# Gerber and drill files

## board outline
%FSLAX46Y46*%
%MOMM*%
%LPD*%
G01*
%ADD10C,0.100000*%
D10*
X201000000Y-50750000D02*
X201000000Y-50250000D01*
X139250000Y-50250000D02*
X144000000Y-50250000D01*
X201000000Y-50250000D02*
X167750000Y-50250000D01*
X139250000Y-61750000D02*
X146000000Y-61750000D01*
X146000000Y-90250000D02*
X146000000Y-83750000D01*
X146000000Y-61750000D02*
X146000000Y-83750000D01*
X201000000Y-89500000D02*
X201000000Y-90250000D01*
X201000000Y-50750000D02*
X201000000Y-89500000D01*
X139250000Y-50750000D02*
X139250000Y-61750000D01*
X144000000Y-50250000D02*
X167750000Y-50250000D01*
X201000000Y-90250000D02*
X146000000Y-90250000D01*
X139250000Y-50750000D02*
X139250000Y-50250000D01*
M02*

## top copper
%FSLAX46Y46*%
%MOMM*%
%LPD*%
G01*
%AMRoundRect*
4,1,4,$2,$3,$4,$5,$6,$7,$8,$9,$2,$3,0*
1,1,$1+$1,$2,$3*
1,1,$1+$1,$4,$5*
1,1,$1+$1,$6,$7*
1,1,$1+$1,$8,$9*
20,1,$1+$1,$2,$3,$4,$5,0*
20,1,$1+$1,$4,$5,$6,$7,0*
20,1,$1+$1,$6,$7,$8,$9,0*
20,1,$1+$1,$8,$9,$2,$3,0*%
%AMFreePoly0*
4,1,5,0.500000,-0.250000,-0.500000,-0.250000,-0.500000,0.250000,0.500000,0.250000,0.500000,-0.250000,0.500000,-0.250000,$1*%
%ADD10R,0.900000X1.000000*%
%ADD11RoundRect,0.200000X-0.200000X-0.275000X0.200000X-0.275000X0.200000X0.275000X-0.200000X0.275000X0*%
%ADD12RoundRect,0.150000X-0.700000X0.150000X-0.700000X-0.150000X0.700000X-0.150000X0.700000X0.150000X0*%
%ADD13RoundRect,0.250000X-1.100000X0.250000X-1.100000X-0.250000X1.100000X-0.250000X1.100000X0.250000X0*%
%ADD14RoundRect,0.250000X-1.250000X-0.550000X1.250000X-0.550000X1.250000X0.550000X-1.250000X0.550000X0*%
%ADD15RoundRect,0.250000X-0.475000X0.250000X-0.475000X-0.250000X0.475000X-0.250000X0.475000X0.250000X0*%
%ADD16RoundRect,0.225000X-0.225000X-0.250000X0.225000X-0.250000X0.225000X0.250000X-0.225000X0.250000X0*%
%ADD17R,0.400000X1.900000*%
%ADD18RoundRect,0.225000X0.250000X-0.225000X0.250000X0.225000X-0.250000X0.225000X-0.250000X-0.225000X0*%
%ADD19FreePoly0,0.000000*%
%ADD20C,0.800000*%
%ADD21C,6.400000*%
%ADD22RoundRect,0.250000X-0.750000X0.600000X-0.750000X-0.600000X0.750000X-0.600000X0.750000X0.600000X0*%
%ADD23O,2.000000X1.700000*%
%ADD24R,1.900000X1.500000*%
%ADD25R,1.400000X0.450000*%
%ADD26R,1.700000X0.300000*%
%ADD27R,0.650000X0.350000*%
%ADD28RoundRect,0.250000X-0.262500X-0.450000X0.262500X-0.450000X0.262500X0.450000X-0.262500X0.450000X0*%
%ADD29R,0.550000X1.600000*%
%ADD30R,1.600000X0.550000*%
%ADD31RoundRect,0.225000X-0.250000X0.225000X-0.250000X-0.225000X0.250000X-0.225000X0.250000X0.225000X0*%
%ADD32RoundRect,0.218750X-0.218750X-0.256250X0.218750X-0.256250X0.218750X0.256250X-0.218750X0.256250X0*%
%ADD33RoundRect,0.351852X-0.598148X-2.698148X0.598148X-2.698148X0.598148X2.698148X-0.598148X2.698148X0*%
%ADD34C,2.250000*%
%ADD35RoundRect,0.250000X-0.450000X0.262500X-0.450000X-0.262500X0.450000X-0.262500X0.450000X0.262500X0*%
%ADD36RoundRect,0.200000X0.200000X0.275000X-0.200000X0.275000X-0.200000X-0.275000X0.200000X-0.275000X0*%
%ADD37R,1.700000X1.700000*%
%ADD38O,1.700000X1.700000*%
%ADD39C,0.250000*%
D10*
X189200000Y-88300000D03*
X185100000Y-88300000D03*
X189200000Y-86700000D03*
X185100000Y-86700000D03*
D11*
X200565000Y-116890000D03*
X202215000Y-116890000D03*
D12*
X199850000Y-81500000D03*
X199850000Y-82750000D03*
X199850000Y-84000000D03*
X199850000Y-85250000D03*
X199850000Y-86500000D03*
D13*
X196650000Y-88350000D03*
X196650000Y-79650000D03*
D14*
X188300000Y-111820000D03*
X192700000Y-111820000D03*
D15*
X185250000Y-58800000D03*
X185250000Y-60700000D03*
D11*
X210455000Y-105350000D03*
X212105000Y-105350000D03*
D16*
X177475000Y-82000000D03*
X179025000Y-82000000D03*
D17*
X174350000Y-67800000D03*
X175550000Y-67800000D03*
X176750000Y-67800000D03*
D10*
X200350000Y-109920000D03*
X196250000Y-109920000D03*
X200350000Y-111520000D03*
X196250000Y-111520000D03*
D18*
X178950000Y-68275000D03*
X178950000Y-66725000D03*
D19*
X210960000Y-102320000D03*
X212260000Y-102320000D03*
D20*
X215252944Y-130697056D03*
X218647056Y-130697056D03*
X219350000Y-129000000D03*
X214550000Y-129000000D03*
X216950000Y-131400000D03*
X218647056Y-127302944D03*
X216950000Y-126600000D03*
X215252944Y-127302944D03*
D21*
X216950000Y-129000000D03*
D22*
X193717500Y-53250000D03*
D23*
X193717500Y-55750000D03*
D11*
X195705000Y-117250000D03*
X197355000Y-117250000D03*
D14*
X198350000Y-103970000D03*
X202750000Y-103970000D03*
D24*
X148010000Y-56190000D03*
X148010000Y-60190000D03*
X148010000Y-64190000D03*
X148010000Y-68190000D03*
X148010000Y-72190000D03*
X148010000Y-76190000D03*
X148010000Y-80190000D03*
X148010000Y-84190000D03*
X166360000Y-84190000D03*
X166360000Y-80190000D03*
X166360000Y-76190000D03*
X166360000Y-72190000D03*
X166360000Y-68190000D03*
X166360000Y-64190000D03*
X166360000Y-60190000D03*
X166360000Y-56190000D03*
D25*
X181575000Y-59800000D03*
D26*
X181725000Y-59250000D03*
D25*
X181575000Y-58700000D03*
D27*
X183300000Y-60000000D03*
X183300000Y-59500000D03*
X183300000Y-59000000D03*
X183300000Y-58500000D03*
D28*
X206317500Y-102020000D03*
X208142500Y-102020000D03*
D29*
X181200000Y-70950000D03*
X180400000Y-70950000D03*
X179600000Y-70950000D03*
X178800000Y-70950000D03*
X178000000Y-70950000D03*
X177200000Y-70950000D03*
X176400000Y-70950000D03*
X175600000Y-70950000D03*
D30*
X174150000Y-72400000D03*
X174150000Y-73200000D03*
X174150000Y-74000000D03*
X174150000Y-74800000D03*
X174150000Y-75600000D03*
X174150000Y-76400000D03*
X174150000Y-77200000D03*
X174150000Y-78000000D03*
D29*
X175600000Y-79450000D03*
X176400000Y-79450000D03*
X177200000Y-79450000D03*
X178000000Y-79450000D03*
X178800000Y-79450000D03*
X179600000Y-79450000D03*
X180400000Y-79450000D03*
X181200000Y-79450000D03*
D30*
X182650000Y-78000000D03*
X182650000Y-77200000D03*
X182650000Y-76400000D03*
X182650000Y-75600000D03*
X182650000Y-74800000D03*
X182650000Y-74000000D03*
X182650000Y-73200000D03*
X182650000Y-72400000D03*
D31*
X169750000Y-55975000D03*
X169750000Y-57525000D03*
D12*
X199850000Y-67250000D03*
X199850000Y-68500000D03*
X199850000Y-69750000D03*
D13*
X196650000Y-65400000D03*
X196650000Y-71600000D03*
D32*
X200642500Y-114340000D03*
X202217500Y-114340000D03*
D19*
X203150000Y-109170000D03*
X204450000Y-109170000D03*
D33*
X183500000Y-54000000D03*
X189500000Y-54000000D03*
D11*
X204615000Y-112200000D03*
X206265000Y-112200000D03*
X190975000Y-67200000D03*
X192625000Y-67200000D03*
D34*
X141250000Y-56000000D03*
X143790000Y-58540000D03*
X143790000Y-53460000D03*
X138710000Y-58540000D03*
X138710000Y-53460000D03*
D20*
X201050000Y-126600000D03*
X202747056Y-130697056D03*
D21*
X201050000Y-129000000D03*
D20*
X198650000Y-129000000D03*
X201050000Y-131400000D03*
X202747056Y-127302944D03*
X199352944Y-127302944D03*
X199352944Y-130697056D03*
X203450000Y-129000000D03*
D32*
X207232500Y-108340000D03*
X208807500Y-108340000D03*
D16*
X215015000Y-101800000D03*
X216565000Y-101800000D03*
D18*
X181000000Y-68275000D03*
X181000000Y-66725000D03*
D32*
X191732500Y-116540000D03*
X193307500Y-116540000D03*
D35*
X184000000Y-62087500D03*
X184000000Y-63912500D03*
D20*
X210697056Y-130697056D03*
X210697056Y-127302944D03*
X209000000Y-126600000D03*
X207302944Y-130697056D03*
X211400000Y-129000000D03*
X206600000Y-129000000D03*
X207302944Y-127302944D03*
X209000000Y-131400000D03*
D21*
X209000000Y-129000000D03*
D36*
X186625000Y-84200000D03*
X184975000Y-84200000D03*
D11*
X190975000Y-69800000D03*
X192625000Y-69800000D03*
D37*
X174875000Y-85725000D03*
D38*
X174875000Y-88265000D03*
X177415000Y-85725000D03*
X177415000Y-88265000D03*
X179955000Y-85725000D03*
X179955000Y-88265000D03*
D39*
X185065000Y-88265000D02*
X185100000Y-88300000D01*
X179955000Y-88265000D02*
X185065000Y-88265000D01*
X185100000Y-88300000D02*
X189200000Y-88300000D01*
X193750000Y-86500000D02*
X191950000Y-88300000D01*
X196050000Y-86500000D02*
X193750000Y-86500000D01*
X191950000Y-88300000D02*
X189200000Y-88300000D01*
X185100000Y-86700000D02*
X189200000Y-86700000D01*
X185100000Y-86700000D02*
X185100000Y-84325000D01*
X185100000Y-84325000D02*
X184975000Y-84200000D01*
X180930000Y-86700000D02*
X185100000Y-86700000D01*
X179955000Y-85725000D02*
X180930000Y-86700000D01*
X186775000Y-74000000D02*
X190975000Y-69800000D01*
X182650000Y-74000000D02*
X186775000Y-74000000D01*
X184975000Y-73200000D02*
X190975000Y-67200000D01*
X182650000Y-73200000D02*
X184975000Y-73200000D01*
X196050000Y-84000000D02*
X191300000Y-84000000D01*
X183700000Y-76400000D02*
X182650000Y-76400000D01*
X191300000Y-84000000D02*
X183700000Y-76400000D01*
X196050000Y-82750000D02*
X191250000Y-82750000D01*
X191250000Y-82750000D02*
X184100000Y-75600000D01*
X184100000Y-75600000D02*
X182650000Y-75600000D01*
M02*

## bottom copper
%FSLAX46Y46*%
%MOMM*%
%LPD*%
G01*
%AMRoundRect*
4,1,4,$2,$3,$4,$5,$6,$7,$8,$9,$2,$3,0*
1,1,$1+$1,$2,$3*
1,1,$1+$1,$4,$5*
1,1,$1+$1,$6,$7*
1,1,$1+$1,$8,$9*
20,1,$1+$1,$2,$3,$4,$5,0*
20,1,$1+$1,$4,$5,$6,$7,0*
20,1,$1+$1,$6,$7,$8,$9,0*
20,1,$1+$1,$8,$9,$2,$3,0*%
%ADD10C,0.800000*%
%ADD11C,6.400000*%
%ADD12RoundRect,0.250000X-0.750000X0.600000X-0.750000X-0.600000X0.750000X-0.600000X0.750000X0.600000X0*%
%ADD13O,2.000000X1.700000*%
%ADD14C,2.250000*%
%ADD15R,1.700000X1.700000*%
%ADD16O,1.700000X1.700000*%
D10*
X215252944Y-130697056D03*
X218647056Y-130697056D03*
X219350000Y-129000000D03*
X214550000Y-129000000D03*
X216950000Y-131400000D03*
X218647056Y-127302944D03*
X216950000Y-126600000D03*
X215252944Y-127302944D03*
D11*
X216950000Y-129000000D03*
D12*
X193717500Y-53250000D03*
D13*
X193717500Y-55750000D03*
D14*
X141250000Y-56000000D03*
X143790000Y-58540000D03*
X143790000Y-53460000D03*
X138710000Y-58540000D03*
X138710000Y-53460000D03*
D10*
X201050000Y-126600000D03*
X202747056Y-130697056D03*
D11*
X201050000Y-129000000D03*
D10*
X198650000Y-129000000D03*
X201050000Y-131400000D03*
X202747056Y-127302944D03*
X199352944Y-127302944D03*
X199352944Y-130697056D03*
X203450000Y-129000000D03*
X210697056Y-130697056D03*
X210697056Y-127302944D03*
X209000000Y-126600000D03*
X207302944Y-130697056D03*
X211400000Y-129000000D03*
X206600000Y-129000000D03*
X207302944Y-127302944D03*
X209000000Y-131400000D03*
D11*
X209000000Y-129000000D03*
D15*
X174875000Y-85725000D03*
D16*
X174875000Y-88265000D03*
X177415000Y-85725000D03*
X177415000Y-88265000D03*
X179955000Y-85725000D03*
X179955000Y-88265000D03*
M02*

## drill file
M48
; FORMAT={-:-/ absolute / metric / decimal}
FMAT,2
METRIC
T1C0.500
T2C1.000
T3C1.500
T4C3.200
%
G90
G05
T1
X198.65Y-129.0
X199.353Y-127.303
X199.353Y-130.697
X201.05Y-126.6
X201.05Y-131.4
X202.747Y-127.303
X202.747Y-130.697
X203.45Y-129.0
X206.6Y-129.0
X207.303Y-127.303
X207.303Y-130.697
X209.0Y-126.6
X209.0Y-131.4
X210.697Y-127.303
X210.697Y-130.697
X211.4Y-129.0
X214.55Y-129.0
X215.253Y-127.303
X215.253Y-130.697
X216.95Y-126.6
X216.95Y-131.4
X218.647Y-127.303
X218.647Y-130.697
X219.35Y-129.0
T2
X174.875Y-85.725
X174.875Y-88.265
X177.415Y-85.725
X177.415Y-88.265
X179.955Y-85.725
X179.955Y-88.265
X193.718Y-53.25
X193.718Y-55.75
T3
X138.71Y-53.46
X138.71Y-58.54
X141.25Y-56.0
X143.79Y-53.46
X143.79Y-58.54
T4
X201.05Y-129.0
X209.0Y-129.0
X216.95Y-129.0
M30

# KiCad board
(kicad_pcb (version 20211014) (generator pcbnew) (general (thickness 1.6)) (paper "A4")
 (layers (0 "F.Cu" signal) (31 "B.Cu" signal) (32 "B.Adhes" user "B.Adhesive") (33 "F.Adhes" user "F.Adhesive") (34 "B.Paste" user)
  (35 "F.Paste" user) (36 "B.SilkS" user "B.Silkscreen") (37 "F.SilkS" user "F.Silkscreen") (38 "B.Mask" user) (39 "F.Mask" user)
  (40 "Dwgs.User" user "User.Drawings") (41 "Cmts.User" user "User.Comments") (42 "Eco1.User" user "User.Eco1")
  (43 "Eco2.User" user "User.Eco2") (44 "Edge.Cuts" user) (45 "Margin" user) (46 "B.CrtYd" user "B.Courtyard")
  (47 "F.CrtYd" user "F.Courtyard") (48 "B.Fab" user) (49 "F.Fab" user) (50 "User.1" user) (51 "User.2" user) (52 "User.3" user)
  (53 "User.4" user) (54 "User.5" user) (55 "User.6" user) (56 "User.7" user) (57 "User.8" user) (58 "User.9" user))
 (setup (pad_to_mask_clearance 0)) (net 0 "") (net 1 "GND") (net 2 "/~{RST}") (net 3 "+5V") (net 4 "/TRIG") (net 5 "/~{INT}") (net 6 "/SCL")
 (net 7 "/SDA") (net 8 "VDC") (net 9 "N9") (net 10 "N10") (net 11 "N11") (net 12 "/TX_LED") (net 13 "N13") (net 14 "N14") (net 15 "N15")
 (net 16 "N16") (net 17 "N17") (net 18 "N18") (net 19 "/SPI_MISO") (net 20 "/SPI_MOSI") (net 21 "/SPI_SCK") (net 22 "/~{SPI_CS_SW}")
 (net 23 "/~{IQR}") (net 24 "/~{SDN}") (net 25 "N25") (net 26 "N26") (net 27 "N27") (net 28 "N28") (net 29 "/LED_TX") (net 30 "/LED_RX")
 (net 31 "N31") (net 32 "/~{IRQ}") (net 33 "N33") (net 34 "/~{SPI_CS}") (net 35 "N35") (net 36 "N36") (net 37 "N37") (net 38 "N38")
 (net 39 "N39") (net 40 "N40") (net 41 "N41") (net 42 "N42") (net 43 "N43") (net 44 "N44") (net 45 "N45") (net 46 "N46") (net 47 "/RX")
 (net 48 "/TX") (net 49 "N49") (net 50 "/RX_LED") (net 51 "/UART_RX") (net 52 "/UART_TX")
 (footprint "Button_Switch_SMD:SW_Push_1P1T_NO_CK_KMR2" (layer "F.Cu") (at 187.15 87.5 180)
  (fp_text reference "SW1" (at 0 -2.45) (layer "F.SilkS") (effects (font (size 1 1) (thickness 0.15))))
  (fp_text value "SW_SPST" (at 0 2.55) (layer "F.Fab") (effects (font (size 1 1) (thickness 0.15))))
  (pad "1" smd rect (at -2.05 -0.8 180) (size 0.9 1) (layers "F.Cu" "F.Paste" "F.Mask") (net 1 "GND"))
  (pad "1" smd rect (at 2.05 -0.8 180) (size 0.9 1) (layers "F.Cu" "F.Paste" "F.Mask") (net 1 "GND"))
  (pad "2" smd rect (at -2.05 0.8 180) (size 0.9 1) (layers "F.Cu" "F.Paste" "F.Mask") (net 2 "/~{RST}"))
  (pad "2" smd rect (at 2.05 0.8 180) (size 0.9 1) (layers "F.Cu" "F.Paste" "F.Mask") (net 2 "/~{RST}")))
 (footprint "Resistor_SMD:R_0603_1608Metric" (layer "F.Cu") (at 201.39 116.89)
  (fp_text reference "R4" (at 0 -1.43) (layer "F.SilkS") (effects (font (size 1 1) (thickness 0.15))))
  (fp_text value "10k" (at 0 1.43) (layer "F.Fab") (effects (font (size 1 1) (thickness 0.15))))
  (pad "1" smd roundrect (at -0.825 0) (size 0.8 0.95) (layers "F.Cu" "F.Paste" "F.Mask") (roundrect_rratio 0.25) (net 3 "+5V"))
  (pad "2" smd roundrect (at 0.825 0) (size 0.8 0.95) (layers "F.Cu" "F.Paste" "F.Mask") (roundrect_rratio 0.25) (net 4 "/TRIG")))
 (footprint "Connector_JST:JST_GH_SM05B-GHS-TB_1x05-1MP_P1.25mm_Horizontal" (layer "F.Cu") (at 198 84 -90)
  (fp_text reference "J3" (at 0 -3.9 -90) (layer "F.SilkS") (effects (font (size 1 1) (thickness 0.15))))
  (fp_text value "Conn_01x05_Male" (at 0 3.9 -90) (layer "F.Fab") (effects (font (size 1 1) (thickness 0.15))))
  (pad "1" smd roundrect (at -2.5 -1.85 270) (size 0.6 1.7) (layers "F.Cu" "F.Paste" "F.Mask") (roundrect_rratio 0.25) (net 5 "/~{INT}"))
  (pad "2" smd roundrect (at -1.25 -1.85 270) (size 0.6 1.7) (layers "F.Cu" "F.Paste" "F.Mask") (roundrect_rratio 0.25) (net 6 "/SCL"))
  (pad "3" smd roundrect (at 0 -1.85 270) (size 0.6 1.7) (layers "F.Cu" "F.Paste" "F.Mask") (roundrect_rratio 0.25) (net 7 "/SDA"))
  (pad "4" smd roundrect (at 1.25 -1.85 270) (size 0.6 1.7) (layers "F.Cu" "F.Paste" "F.Mask") (roundrect_rratio 0.25) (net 3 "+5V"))
  (pad "5" smd roundrect (at 2.5 -1.85 270) (size 0.6 1.7) (layers "F.Cu" "F.Paste" "F.Mask") (roundrect_rratio 0.25) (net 1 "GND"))
  (pad "MP" smd roundrect (at 4.35 1.35 270) (size 1 2.7) (layers "F.Cu" "F.Paste" "F.Mask") (roundrect_rratio 0.25))
  (pad "MP" smd roundrect (at -4.35 1.35 270) (size 1 2.7) (layers "F.Cu" "F.Paste" "F.Mask") (roundrect_rratio 0.25)))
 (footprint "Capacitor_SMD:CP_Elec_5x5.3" (layer "F.Cu") (at 190.5 111.82)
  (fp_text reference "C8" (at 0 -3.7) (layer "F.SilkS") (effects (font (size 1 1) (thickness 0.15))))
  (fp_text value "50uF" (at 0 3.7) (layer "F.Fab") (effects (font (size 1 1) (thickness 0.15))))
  (pad "1" smd roundrect (at -2.2 0) (size 3 1.6) (layers "F.Cu" "F.Paste" "F.Mask") (roundrect_rratio 0.15625) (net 3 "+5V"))
  (pad "2" smd roundrect (at 2.2 0) (size 3 1.6) (layers "F.Cu" "F.Paste" "F.Mask") (roundrect_rratio 0.15625) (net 1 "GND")))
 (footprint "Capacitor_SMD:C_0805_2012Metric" (layer "F.Cu") (at 185.25 59.75 -90)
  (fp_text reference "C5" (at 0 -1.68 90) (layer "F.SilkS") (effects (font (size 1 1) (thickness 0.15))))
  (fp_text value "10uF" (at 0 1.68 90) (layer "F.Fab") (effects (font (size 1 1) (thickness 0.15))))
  (pad "1" smd roundrect (at -0.95 0 270) (size 1 1.45) (layers "F.Cu" "F.Paste" "F.Mask") (roundrect_rratio 0.25) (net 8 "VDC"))
  (pad "2" smd roundrect (at 0.95 0 270) (size 1 1.45) (layers "F.Cu" "F.Paste" "F.Mask") (roundrect_rratio 0.25) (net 1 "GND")))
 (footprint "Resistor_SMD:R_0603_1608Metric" (layer "F.Cu") (at 211.28 105.35)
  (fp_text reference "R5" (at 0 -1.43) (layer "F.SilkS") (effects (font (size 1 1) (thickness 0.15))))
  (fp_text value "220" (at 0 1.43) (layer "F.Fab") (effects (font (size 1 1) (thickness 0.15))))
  (pad "1" smd roundrect (at -0.825 0) (size 0.8 0.95) (layers "F.Cu" "F.Paste" "F.Mask") (roundrect_rratio 0.25) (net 3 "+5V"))
  (pad "2" smd roundrect (at 0.825 0) (size 0.8 0.95) (layers "F.Cu" "F.Paste" "F.Mask") (roundrect_rratio 0.25) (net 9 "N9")))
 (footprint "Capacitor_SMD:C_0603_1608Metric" (layer "F.Cu") (at 178.25 82)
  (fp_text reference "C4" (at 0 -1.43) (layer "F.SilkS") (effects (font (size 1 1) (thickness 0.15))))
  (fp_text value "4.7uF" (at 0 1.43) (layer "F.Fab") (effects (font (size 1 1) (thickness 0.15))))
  (pad "1" smd roundrect (at -0.775 0) (size 0.9 0.95) (layers "F.Cu" "F.Paste" "F.Mask") (roundrect_rratio 0.25) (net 3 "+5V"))
  (pad "2" smd roundrect (at 0.775 0) (size 0.9 0.95) (layers "F.Cu" "F.Paste" "F.Mask") (roundrect_rratio 0.25) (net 1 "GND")))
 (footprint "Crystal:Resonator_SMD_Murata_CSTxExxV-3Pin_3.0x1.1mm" (layer "F.Cu") (at 175.55 67.8)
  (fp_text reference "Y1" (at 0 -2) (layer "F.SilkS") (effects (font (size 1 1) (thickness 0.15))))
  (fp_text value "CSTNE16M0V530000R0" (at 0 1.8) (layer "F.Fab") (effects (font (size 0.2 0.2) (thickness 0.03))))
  (pad "1" smd rect (at -1.2 0) (size 0.4 1.9) (layers "F.Cu" "F.Paste" "F.Mask") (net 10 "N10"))
  (pad "2" smd rect (at 0 0) (size 0.4 1.9) (layers "F.Cu" "F.Paste" "F.Mask") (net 1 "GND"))
  (pad "3" smd rect (at 1.2 0) (size 0.4 1.9) (layers "F.Cu" "F.Paste" "F.Mask") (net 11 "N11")))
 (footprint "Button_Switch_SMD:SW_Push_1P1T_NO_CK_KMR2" (layer "F.Cu") (at 198.3 110.72)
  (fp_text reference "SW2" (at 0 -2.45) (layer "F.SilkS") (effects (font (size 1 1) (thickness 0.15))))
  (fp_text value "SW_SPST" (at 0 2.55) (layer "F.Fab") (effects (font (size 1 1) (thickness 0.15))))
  (pad "1" smd rect (at 2.05 -0.8) (size 0.9 1) (layers "F.Cu" "F.Paste" "F.Mask") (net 1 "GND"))
  (pad "1" smd rect (at -2.05 -0.8) (size 0.9 1) (layers "F.Cu" "F.Paste" "F.Mask") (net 1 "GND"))
  (pad "2" smd rect (at 2.05 0.8) (size 0.9 1) (layers "F.Cu" "F.Paste" "F.Mask") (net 4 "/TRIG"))
  (pad "2" smd rect (at -2.05 0.8) (size 0.9 1) (layers "F.Cu" "F.Paste" "F.Mask") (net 4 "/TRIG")))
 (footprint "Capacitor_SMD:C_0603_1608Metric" (layer "F.Cu") (at 178.95 67.5 90)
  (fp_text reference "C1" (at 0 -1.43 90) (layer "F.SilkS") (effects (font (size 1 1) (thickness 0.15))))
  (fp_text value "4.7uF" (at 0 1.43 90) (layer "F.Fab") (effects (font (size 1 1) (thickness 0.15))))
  (pad "1" smd roundrect (at -0.775 0 90) (size 0.9 0.95) (layers "F.Cu" "F.Paste" "F.Mask") (roundrect_rratio 0.25) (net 3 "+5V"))
  (pad "2" smd roundrect (at 0.775 0 90) (size 0.9 0.95) (layers "F.Cu" "F.Paste" "F.Mask") (roundrect_rratio 0.25) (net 1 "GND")))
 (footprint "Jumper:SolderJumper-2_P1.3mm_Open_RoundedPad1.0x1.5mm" (layer "F.Cu") (at 211.61 102.32)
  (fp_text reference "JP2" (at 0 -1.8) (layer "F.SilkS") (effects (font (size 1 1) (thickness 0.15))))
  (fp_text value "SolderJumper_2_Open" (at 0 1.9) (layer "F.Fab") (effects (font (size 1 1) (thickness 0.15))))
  (pad "1" smd custom (at -0.65 0) (size 1 0.5) (layers "F.Cu" "F.Mask") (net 3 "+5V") (zone_connect 2)
   (options (clearance outline) (anchor rect)) (primitives))
  (pad "2" smd custom (at 0.65 0) (size 1 0.5) (layers "F.Cu" "F.Mask") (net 8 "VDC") (zone_connect 2)
   (options (clearance outline) (anchor rect)) (primitives)))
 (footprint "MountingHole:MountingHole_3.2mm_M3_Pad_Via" (layer "F.Cu") (at 216.95 129)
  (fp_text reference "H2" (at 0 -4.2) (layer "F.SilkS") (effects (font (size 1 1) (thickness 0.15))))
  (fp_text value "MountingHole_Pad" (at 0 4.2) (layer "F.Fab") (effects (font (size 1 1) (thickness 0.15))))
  (pad "1" thru_hole circle (at -1.697056 1.697056) (size 0.8 0.8) (drill 0.5) (layers *.Cu *.Mask) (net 1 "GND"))
  (pad "1" thru_hole circle (at 1.697056 1.697056) (size 0.8 0.8) (drill 0.5) (layers *.Cu *.Mask) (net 1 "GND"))
  (pad "1" thru_hole circle (at 2.4 0) (size 0.8 0.8) (drill 0.5) (layers *.Cu *.Mask) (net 1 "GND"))
  (pad "1" thru_hole circle (at -2.4 0) (size 0.8 0.8) (drill 0.5) (layers *.Cu *.Mask) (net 1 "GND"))
  (pad "1" thru_hole circle (at 0 2.4) (size 0.8 0.8) (drill 0.5) (layers *.Cu *.Mask) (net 1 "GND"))
  (pad "1" thru_hole circle (at 1.697056 -1.697056) (size 0.8 0.8) (drill 0.5) (layers *.Cu *.Mask) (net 1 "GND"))
  (pad "1" thru_hole circle (at 0 -2.4) (size 0.8 0.8) (drill 0.5) (layers *.Cu *.Mask) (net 1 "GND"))
  (pad "1" thru_hole circle (at -1.697056 -1.697056) (size 0.8 0.8) (drill 0.5) (layers *.Cu *.Mask) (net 1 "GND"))
  (pad "1" thru_hole circle (at 0 0) (size 6.4 6.4) (drill 3.2) (layers *.Cu *.Mask) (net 1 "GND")))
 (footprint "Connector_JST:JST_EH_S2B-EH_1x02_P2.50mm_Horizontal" (layer "F.Cu") (at 193.7175 53.25 -90)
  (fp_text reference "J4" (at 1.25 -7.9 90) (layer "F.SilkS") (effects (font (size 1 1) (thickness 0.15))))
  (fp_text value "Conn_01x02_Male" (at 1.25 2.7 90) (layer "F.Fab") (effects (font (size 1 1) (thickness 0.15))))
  (pad "1" thru_hole roundrect (at 0 0 270) (size 1.7 2) (drill 1) (layers *.Cu *.Mask) (roundrect_rratio 0.147059) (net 3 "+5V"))
  (pad "2" thru_hole oval (at 2.5 0 270) (size 1.7 2) (drill 1) (layers *.Cu *.Mask) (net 1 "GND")))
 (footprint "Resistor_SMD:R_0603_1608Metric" (layer "F.Cu") (at 196.53 117.25)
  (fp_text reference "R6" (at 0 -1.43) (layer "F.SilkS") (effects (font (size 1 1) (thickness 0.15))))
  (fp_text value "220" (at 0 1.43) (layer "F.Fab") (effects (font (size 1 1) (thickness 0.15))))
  (pad "1" smd roundrect (at -0.825 0) (size 0.8 0.95) (layers "F.Cu" "F.Paste" "F.Mask") (roundrect_rratio 0.25) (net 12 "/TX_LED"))
  (pad "2" smd roundrect (at 0.825 0) (size 0.8 0.95) (layers "F.Cu" "F.Paste" "F.Mask") (roundrect_rratio 0.25) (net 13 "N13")))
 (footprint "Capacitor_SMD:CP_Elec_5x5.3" (layer "F.Cu") (at 200.55 103.97)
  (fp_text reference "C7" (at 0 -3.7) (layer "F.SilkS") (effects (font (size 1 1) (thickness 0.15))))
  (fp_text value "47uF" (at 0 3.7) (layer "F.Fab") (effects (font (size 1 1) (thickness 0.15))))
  (pad "1" smd roundrect (at -2.2 0) (size 3 1.6) (layers "F.Cu" "F.Paste" "F.Mask") (roundrect_rratio 0.15625) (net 3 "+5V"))
  (pad "2" smd roundrect (at 2.2 0) (size 3 1.6) (layers "F.Cu" "F.Paste" "F.Mask") (roundrect_rratio 0.15625) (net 1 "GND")))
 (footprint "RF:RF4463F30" (layer "F.Cu") (at 157.21 70.19)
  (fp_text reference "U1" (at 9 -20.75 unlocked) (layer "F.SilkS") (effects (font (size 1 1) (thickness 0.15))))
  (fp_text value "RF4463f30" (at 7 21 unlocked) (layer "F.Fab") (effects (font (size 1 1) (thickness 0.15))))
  (pad "1" smd rect (at -9.2 -14 270) (size 1.5 1.9) (layers "F.Cu" "F.Paste" "F.Mask") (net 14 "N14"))
  (pad "2" smd rect (at -9.2 -10 270) (size 1.5 1.9) (layers "F.Cu" "F.Paste" "F.Mask") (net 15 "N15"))
  (pad "3" smd rect (at -9.2 -6 90) (size 1.5 1.9) (layers "F.Cu" "F.Paste" "F.Mask") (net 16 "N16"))
  (pad "4" smd rect (at -9.2 -2 90) (size 1.5 1.9) (layers "F.Cu" "F.Paste" "F.Mask") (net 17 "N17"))
  (pad "5" smd rect (at -9.2 2 270) (size 1.5 1.9) (layers "F.Cu" "F.Paste" "F.Mask") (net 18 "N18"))
  (pad "6" smd rect (at -9.2 6 90) (size 1.5 1.9) (layers "F.Cu" "F.Paste" "F.Mask") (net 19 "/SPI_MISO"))
  (pad "7" smd rect (at -9.2 10 90) (size 1.5 1.9) (layers "F.Cu" "F.Paste" "F.Mask") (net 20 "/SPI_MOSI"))
  (pad "8" smd rect (at -9.2 14 90) (size 1.5 1.9) (layers "F.Cu" "F.Paste" "F.Mask") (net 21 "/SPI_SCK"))
  (pad "9" smd rect (at 9.15 14 90) (size 1.5 1.9) (layers "F.Cu" "F.Paste" "F.Mask") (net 1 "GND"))
  (pad "10" smd rect (at 9.15 10 90) (size 1.5 1.9) (layers "F.Cu" "F.Paste" "F.Mask") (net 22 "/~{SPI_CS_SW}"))
  (pad "11" smd rect (at 9.15 6 90) (size 1.5 1.9) (layers "F.Cu" "F.Paste" "F.Mask") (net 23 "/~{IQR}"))
  (pad "12" smd rect (at 9.15 2 90) (size 1.5 1.9) (layers "F.Cu" "F.Paste" "F.Mask") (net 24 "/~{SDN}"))
  (pad "13" smd rect (at 9.15 -2 90) (size 1.5 1.9) (layers "F.Cu" "F.Paste" "F.Mask") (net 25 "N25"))
  (pad "14" smd rect (at 9.15 -6 90) (size 1.5 1.9) (layers "F.Cu" "F.Paste" "F.Mask") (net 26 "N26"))
  (pad "15" smd rect (at 9.15 -10 90) (size 1.5 1.9) (layers "F.Cu" "F.Paste" "F.Mask") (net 1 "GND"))
  (pad "16" smd rect (at 9.15 -14 90) (size 1.5 1.9) (layers "F.Cu" "F.Paste" "F.Mask") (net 3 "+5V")))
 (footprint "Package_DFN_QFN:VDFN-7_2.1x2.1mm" (layer "F.Cu") (at 182.25 59.25)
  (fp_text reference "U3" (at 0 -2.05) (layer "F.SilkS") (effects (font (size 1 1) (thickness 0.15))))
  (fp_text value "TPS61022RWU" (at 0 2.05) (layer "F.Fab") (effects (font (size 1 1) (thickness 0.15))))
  (pad "1" smd rect (at -0.675 0.55) (size 1.4 0.45) (layers "F.Cu" "F.Paste" "F.Mask") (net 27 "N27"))
  (pad "2" smd rect (at -0.525 0) (size 1.7 0.3) (layers "F.Cu" "F.Paste" "F.Mask") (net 8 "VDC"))
  (pad "3" smd rect (at -0.675 -0.55) (size 1.4 0.45) (layers "F.Cu" "F.Paste" "F.Mask") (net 1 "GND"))
  (pad "5" smd rect (at 1.05 0.75) (size 0.65 0.35) (layers "F.Cu" "F.Paste" "F.Mask") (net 1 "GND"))
  (pad "6" smd rect (at 1.05 0.25) (size 0.65 0.35) (layers "F.Cu" "F.Paste" "F.Mask") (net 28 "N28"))
  (pad "7" smd rect (at 1.05 -0.25) (size 0.65 0.35) (layers "F.Cu" "F.Paste" "F.Mask") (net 3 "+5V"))
  (pad "8" smd rect (at 1.05 -0.75) (size 0.65 0.35) (layers "F.Cu" "F.Paste" "F.Mask")))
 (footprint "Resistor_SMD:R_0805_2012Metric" (layer "F.Cu") (at 207.23 102.02)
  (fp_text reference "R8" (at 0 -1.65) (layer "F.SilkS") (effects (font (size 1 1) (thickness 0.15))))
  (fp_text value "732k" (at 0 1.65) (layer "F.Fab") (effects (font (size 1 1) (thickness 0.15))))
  (pad "1" smd roundrect (at -0.9125 0) (size 1.025 1.4) (layers "F.Cu" "F.Paste" "F.Mask") (roundrect_rratio 0.243902) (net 3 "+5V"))
  (pad "2" smd roundrect (at 0.9125 0) (size 1.025 1.4) (layers "F.Cu" "F.Paste" "F.Mask") (roundrect_rratio 0.243902) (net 27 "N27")))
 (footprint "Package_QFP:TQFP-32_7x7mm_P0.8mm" (layer "F.Cu") (at 178.4 75.2 -90)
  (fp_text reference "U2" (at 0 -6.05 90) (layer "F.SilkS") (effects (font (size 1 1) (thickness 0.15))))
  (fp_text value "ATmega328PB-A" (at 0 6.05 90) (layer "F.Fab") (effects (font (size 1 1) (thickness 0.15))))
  (pad "1" smd rect (at -4.25 -2.8 270) (size 1.6 0.55) (layers "F.Cu" "F.Paste" "F.Mask") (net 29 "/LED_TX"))
  (pad "2" smd rect (at -4.25 -2 270) (size 1.6 0.55) (layers "F.Cu" "F.Paste" "F.Mask") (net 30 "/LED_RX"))
  (pad "3" smd rect (at -4.25 -1.2 270) (size 1.6 0.55) (layers "F.Cu" "F.Paste" "F.Mask") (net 20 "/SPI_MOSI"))
  (pad "4" smd rect (at -4.25 -0.4 270) (size 1.6 0.55) (layers "F.Cu" "F.Paste" "F.Mask") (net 3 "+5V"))
  (pad "5" smd rect (at -4.25 0.4 270) (size 1.6 0.55) (layers "F.Cu" "F.Paste" "F.Mask") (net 1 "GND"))
  (pad "6" smd rect (at -4.25 1.2 270) (size 1.6 0.55) (layers "F.Cu" "F.Paste" "F.Mask") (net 19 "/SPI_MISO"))
  (pad "7" smd rect (at -4.25 2 270) (size 1.6 0.55) (layers "F.Cu" "F.Paste" "F.Mask") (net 11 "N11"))
  (pad "8" smd rect (at -4.25 2.8 270) (size 1.6 0.55) (layers "F.Cu" "F.Paste" "F.Mask") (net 10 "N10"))
  (pad "9" smd rect (at -2.8 4.25) (size 1.6 0.55) (layers "F.Cu" "F.Paste" "F.Mask") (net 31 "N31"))
  (pad "10" smd rect (at -2 4.25) (size 1.6 0.55) (layers "F.Cu" "F.Paste" "F.Mask") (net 24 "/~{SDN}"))
  (pad "11" smd rect (at -1.2 4.25) (size 1.6 0.55) (layers "F.Cu" "F.Paste" "F.Mask") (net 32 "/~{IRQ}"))
  (pad "12" smd rect (at -0.4 4.25) (size 1.6 0.55) (layers "F.Cu" "F.Paste" "F.Mask") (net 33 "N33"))
  (pad "13" smd rect (at 0.4 4.25) (size 1.6 0.55) (layers "F.Cu" "F.Paste" "F.Mask") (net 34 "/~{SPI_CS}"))
  (pad "14" smd rect (at 1.2 4.25) (size 1.6 0.55) (layers "F.Cu" "F.Paste" "F.Mask") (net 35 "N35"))
  (pad "15" smd rect (at 2 4.25) (size 1.6 0.55) (layers "F.Cu" "F.Paste" "F.Mask") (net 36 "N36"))
  (pad "16" smd rect (at 2.8 4.25) (size 1.6 0.55) (layers "F.Cu" "F.Paste" "F.Mask") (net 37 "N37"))
  (pad "17" smd rect (at 4.25 2.8 270) (size 1.6 0.55) (layers "F.Cu" "F.Paste" "F.Mask") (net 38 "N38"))
  (pad "18" smd rect (at 4.25 2 270) (size 1.6 0.55) (layers "F.Cu" "F.Paste" "F.Mask") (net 3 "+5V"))
  (pad "19" smd rect (at 4.25 1.2 270) (size 1.6 0.55) (layers "F.Cu" "F.Paste" "F.Mask") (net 21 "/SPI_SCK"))
  (pad "20" smd rect (at 4.25 0.4 270) (size 1.6 0.55) (layers "F.Cu" "F.Paste" "F.Mask") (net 3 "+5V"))
  (pad "21" smd rect (at 4.25 -0.4 270) (size 1.6 0.55) (layers "F.Cu" "F.Paste" "F.Mask") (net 1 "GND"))
  (pad "22" smd rect (at 4.25 -1.2 270) (size 1.6 0.55) (layers "F.Cu" "F.Paste" "F.Mask") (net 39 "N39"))
  (pad "23" smd rect (at 4.25 -2 270) (size 1.6 0.55) (layers "F.Cu" "F.Paste" "F.Mask") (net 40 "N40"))
  (pad "24" smd rect (at 4.25 -2.8 270) (size 1.6 0.55) (layers "F.Cu" "F.Paste" "F.Mask") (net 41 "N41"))
  (pad "25" smd rect (at 2.8 -4.25) (size 1.6 0.55) (layers "F.Cu" "F.Paste" "F.Mask") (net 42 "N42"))
  (pad "26" smd rect (at 2 -4.25) (size 1.6 0.55) (layers "F.Cu" "F.Paste" "F.Mask") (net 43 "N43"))
  (pad "27" smd rect (at 1.2 -4.25) (size 1.6 0.55) (layers "F.Cu" "F.Paste" "F.Mask") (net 7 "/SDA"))
  (pad "28" smd rect (at 0.4 -4.25) (size 1.6 0.55) (layers "F.Cu" "F.Paste" "F.Mask") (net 6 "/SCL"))
  (pad "29" smd rect (at -0.4 -4.25) (size 1.6 0.55) (layers "F.Cu" "F.Paste" "F.Mask") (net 2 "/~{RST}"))
  (pad "30" smd rect (at -1.2 -4.25) (size 1.6 0.55) (layers "F.Cu" "F.Paste" "F.Mask") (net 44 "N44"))
  (pad "31" smd rect (at -2 -4.25) (size 1.6 0.55) (layers "F.Cu" "F.Paste" "F.Mask") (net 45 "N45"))
  (pad "32" smd rect (at -2.8 -4.25) (size 1.6 0.55) (layers "F.Cu" "F.Paste" "F.Mask") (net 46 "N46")))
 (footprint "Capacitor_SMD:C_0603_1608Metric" (layer "F.Cu") (at 169.75 56.75 -90)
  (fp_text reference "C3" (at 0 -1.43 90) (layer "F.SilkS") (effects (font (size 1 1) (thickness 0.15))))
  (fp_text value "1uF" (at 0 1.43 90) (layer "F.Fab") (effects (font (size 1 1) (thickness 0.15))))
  (pad "1" smd roundrect (at -0.775 0 270) (size 0.9 0.95) (layers "F.Cu" "F.Paste" "F.Mask") (roundrect_rratio 0.25) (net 3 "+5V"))
  (pad "2" smd roundrect (at 0.775 0 270) (size 0.9 0.95) (layers "F.Cu" "F.Paste" "F.Mask") (roundrect_rratio 0.25) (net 1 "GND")))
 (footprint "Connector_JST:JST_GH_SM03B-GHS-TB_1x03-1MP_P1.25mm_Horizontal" (layer "F.Cu") (at 198 68.5 -90)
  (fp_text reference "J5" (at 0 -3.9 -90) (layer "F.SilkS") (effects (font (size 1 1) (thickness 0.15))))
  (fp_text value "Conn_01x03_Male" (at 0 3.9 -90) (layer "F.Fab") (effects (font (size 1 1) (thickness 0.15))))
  (pad "1" smd roundrect (at -1.25 -1.85 270) (size 0.6 1.7) (layers "F.Cu" "F.Paste" "F.Mask") (roundrect_rratio 0.25) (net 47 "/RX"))
  (pad "2" smd roundrect (at 0 -1.85 270) (size 0.6 1.7) (layers "F.Cu" "F.Paste" "F.Mask") (roundrect_rratio 0.25) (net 1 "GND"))
  (pad "3" smd roundrect (at 1.25 -1.85 270) (size 0.6 1.7) (layers "F.Cu" "F.Paste" "F.Mask") (roundrect_rratio 0.25) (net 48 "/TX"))
  (pad "MP" smd roundrect (at -3.1 1.35 270) (size 1 2.7) (layers "F.Cu" "F.Paste" "F.Mask") (roundrect_rratio 0.25))
  (pad "MP" smd roundrect (at 3.1 1.35 270) (size 1 2.7) (layers "F.Cu" "F.Paste" "F.Mask") (roundrect_rratio 0.25)))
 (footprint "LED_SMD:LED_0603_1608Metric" (layer "F.Cu") (at 201.43 114.34)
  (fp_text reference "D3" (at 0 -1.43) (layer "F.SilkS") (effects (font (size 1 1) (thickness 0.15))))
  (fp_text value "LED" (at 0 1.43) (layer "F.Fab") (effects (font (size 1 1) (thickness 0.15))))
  (pad "1" smd roundrect (at -0.7875 0) (size 0.875 0.95) (layers "F.Cu" "F.Paste" "F.Mask") (roundrect_rratio 0.25) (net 1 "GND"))
  (pad "2" smd roundrect (at 0.7875 0) (size 0.875 0.95) (layers "F.Cu" "F.Paste" "F.Mask") (roundrect_rratio 0.25) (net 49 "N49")))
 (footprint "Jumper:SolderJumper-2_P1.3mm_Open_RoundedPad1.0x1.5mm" (layer "F.Cu") (at 203.8 109.17)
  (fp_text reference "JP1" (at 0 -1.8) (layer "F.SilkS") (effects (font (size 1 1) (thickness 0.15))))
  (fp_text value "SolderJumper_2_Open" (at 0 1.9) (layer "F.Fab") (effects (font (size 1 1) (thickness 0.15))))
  (pad "1" smd custom (at -0.65 0) (size 1 0.5) (layers "F.Cu" "F.Mask") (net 34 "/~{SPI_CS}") (zone_connect 2)
   (options (clearance outline) (anchor rect)) (primitives))
  (pad "2" smd custom (at 0.65 0) (size 1 0.5) (layers "F.Cu" "F.Mask") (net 22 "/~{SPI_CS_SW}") (zone_connect 2)
   (options (clearance outline) (anchor rect)) (primitives)))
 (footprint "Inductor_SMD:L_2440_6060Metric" (layer "F.Cu") (at 186.5 54)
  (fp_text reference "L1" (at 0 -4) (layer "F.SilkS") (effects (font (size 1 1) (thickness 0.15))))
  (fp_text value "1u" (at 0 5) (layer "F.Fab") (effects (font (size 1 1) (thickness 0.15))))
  (pad "1" smd roundrect (at -3 0) (size 1.9 6.1) (layers "F.Cu" "F.Paste" "F.Mask") (roundrect_rratio 0.185185) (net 8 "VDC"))
  (pad "1" smd roundrect (at 3 0) (size 1.9 6.1) (layers "F.Cu" "F.Paste" "F.Mask") (roundrect_rratio 0.185185) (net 8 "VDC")))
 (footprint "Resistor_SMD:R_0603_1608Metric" (layer "F.Cu") (at 205.44 112.2)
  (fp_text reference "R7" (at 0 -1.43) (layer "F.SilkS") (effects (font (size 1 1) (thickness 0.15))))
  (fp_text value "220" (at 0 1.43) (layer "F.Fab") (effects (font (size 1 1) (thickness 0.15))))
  (pad "1" smd roundrect (at -0.825 0) (size 0.8 0.95) (layers "F.Cu" "F.Paste" "F.Mask") (roundrect_rratio 0.25) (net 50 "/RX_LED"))
  (pad "2" smd roundrect (at 0.825 0) (size 0.8 0.95) (layers "F.Cu" "F.Paste" "F.Mask") (roundrect_rratio 0.25) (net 49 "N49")))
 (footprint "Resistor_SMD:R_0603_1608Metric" (layer "F.Cu") (at 191.8 67.2)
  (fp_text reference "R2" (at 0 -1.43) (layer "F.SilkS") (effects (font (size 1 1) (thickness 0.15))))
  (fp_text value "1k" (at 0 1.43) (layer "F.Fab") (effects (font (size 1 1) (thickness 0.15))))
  (pad "1" smd roundrect (at -0.825 0) (size 0.8 0.95) (layers "F.Cu" "F.Paste" "F.Mask") (roundrect_rratio 0.25) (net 45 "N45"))
  (pad "2" smd roundrect (at 0.825 0) (size 0.8 0.95) (layers "F.Cu" "F.Paste" "F.Mask") (roundrect_rratio 0.25) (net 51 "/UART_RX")))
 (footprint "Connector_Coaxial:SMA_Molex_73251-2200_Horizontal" (layer "F.Cu") (at 141.25 56 90)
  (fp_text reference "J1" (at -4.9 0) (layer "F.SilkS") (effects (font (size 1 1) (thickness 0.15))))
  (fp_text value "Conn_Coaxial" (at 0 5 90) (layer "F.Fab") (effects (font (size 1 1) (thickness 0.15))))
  (pad "1" thru_hole circle (at 0 0 90) (size 2.25 2.25) (drill 1.5) (layers *.Cu *.Mask) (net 14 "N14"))
  (pad "2" thru_hole circle (at -2.54 2.54 90) (size 2.25 2.25) (drill 1.5) (layers *.Cu *.Mask) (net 15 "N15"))
  (pad "2" thru_hole circle (at 2.54 2.54 180) (size 2.25 2.25) (drill 1.5) (layers *.Cu *.Mask) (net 15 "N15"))
  (pad "2" thru_hole circle (at -2.54 -2.54 90) (size 2.25 2.25) (drill 1.5) (layers *.Cu *.Mask) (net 15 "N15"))
  (pad "2" thru_hole circle (at 2.54 -2.54 90) (size 2.25 2.25) (drill 1.5) (layers *.Cu *.Mask) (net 15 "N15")))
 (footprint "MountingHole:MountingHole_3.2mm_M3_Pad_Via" (layer "F.Cu") (at 201.05 129)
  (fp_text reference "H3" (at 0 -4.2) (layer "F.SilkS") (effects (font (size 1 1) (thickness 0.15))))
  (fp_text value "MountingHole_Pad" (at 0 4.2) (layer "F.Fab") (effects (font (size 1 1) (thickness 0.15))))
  (pad "1" thru_hole circle (at 0 -2.4) (size 0.8 0.8) (drill 0.5) (layers *.Cu *.Mask) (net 1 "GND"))
  (pad "1" thru_hole circle (at 1.697056 1.697056) (size 0.8 0.8) (drill 0.5) (layers *.Cu *.Mask) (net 1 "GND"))
  (pad "1" thru_hole circle (at 0 0) (size 6.4 6.4) (drill 3.2) (layers *.Cu *.Mask) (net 1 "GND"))
  (pad "1" thru_hole circle (at -2.4 0) (size 0.8 0.8) (drill 0.5) (layers *.Cu *.Mask) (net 1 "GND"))
  (pad "1" thru_hole circle (at 0 2.4) (size 0.8 0.8) (drill 0.5) (layers *.Cu *.Mask) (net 1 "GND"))
  (pad "1" thru_hole circle (at 1.697056 -1.697056) (size 0.8 0.8) (drill 0.5) (layers *.Cu *.Mask) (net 1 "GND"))
  (pad "1" thru_hole circle (at -1.697056 -1.697056) (size 0.8 0.8) (drill 0.5) (layers *.Cu *.Mask) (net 1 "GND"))
  (pad "1" thru_hole circle (at -1.697056 1.697056) (size 0.8 0.8) (drill 0.5) (layers *.Cu *.Mask) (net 1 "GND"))
  (pad "1" thru_hole circle (at 2.4 0) (size 0.8 0.8) (drill 0.5) (layers *.Cu *.Mask) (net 1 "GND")))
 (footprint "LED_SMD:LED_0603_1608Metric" (layer "F.Cu") (at 208.02 108.34)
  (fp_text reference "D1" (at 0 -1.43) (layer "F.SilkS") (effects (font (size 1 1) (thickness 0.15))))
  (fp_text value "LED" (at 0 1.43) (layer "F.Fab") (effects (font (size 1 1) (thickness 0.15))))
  (pad "1" smd roundrect (at -0.7875 0) (size 0.875 0.95) (layers "F.Cu" "F.Paste" "F.Mask") (roundrect_rratio 0.25) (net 1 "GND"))
  (pad "2" smd roundrect (at 0.7875 0) (size 0.875 0.95) (layers "F.Cu" "F.Paste" "F.Mask") (roundrect_rratio 0.25) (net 9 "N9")))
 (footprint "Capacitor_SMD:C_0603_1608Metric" (layer "F.Cu") (at 215.79 101.8)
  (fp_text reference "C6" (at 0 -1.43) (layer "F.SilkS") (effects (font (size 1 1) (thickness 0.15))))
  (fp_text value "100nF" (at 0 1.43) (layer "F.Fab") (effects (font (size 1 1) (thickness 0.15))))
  (pad "1" smd roundrect (at -0.775 0) (size 0.9 0.95) (layers "F.Cu" "F.Paste" "F.Mask") (roundrect_rratio 0.25) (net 3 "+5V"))
  (pad "2" smd roundrect (at 0.775 0) (size 0.9 0.95) (layers "F.Cu" "F.Paste" "F.Mask") (roundrect_rratio 0.25) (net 1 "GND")))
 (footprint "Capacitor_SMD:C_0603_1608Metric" (layer "F.Cu") (at 181 67.5 90)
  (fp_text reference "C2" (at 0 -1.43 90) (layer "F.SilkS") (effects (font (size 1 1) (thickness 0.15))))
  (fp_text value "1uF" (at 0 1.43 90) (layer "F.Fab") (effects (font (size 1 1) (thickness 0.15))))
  (pad "1" smd roundrect (at -0.775 0 90) (size 0.9 0.95) (layers "F.Cu" "F.Paste" "F.Mask") (roundrect_rratio 0.25) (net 3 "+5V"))
  (pad "2" smd roundrect (at 0.775 0 90) (size 0.9 0.95) (layers "F.Cu" "F.Paste" "F.Mask") (roundrect_rratio 0.25) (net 1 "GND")))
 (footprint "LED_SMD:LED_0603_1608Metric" (layer "F.Cu") (at 192.52 116.54)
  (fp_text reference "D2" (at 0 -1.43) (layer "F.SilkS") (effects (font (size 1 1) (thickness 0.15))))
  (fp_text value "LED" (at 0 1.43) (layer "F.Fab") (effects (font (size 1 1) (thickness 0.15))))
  (pad "1" smd roundrect (at -0.7875 0) (size 0.875 0.95) (layers "F.Cu" "F.Paste" "F.Mask") (roundrect_rratio 0.25) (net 1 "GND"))
  (pad "2" smd roundrect (at 0.7875 0) (size 0.875 0.95) (layers "F.Cu" "F.Paste" "F.Mask") (roundrect_rratio 0.25) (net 13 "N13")))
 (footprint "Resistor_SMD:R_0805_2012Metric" (layer "F.Cu") (at 184 63 -90)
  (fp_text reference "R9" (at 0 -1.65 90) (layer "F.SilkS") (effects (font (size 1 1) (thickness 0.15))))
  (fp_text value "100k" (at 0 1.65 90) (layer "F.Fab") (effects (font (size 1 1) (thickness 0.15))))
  (pad "1" smd roundrect (at -0.9125 0 270) (size 1.025 1.4) (layers "F.Cu" "F.Paste" "F.Mask") (roundrect_rratio 0.243902) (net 27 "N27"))
  (pad "2" smd roundrect (at 0.9125 0 270) (size 1.025 1.4) (layers "F.Cu" "F.Paste" "F.Mask") (roundrect_rratio 0.243902) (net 1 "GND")))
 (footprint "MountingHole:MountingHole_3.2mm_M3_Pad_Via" (layer "F.Cu") (at 209 129)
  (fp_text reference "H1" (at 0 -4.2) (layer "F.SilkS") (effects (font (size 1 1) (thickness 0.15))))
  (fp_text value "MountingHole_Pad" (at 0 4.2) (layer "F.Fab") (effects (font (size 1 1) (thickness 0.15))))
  (pad "1" thru_hole circle (at 1.697056 1.697056) (size 0.8 0.8) (drill 0.5) (layers *.Cu *.Mask) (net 1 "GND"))
  (pad "1" thru_hole circle (at 1.697056 -1.697056) (size 0.8 0.8) (drill 0.5) (layers *.Cu *.Mask) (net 1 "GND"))
  (pad "1" thru_hole circle (at 0 -2.4) (size 0.8 0.8) (drill 0.5) (layers *.Cu *.Mask) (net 1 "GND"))
  (pad "1" thru_hole circle (at -1.697056 1.697056) (size 0.8 0.8) (drill 0.5) (layers *.Cu *.Mask) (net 1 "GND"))
  (pad "1" thru_hole circle (at 2.4 0) (size 0.8 0.8) (drill 0.5) (layers *.Cu *.Mask) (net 1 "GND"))
  (pad "1" thru_hole circle (at -2.4 0) (size 0.8 0.8) (drill 0.5) (layers *.Cu *.Mask) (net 1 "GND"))
  (pad "1" thru_hole circle (at -1.697056 -1.697056) (size 0.8 0.8) (drill 0.5) (layers *.Cu *.Mask) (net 1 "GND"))
  (pad "1" thru_hole circle (at 0 2.4) (size 0.8 0.8) (drill 0.5) (layers *.Cu *.Mask) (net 1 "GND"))
  (pad "1" thru_hole circle (at 0 0) (size 6.4 6.4) (drill 3.2) (layers *.Cu *.Mask) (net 1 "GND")))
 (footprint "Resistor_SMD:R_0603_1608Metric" (layer "F.Cu") (at 185.8 84.2 180)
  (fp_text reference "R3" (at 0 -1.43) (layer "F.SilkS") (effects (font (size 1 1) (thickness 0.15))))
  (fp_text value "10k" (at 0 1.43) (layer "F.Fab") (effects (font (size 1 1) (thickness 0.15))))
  (pad "1" smd roundrect (at -0.825 0 180) (size 0.8 0.95) (layers "F.Cu" "F.Paste" "F.Mask") (roundrect_rratio 0.25) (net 3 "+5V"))
  (pad "2" smd roundrect (at 0.825 0 180) (size 0.8 0.95) (layers "F.Cu" "F.Paste" "F.Mask") (roundrect_rratio 0.25) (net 2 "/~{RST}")))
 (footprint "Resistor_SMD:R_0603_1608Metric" (layer "F.Cu") (at 191.8 69.8)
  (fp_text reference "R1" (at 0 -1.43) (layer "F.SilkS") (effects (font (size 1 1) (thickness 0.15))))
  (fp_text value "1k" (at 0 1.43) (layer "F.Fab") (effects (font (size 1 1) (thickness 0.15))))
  (pad "1" smd roundrect (at -0.825 0) (size 0.8 0.95) (layers "F.Cu" "F.Paste" "F.Mask") (roundrect_rratio 0.25) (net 44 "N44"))
  (pad "2" smd roundrect (at 0.825 0) (size 0.8 0.95) (layers "F.Cu" "F.Paste" "F.Mask") (roundrect_rratio 0.25) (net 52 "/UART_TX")))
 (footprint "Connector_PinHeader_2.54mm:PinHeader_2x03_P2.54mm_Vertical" (layer "B.Cu") (at 174.875 85.725 -90)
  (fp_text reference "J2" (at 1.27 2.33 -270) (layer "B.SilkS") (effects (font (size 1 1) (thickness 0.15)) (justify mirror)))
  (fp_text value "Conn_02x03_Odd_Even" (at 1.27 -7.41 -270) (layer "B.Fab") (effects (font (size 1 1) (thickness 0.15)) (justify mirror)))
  (pad "1" thru_hole rect (at 0 0 270) (size 1.7 1.7) (drill 1) (layers *.Cu *.Mask) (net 19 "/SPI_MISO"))
  (pad "2" thru_hole oval (at 2.54 0 270) (size 1.7 1.7) (drill 1) (layers *.Cu *.Mask) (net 3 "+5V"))
  (pad "3" thru_hole oval (at 0 -2.54 270) (size 1.7 1.7) (drill 1) (layers *.Cu *.Mask) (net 21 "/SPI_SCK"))
  (pad "4" thru_hole oval (at 2.54 -2.54 270) (size 1.7 1.7) (drill 1) (layers *.Cu *.Mask) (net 20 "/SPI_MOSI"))
  (pad "5" thru_hole oval (at 0 -5.08 270) (size 1.7 1.7) (drill 1) (layers *.Cu *.Mask) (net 2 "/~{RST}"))
  (pad "6" thru_hole oval (at 2.54 -5.08 270) (size 1.7 1.7) (drill 1) (layers *.Cu *.Mask) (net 1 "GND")))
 (gr_line (start 201 50.75) (end 201 50.25) (layer "Edge.Cuts") (width 0.1))
 (gr_line (start 139.25 50.25) (end 144 50.25) (layer "Edge.Cuts") (width 0.1))
 (gr_line (start 201 50.25) (end 167.75 50.25) (layer "Edge.Cuts") (width 0.1))
 (gr_line (start 139.25 61.75) (end 146 61.75) (layer "Edge.Cuts") (width 0.1))
 (gr_line (start 146 90.25) (end 146 83.75) (layer "Edge.Cuts") (width 0.1))
 (gr_line (start 146 61.75) (end 146 83.75) (layer "Edge.Cuts") (width 0.1))
 (gr_line (start 201 89.5) (end 201 90.25) (layer "Edge.Cuts") (width 0.1))
 (gr_line (start 201 50.75) (end 201 89.5) (layer "Edge.Cuts") (width 0.1))
 (gr_line (start 139.25 50.75) (end 139.25 61.75) (layer "Edge.Cuts") (width 0.1))
 (gr_line (start 144 50.25) (end 167.75 50.25) (layer "Edge.Cuts") (width 0.1))
 (gr_line (start 201 90.25) (end 146 90.25) (layer "Edge.Cuts") (width 0.1))
 (gr_line (start 139.25 50.75) (end 139.25 50.25) (layer "Edge.Cuts") (width 0.1))
 (segment (start 185.065 88.265) (end 185.1 88.3) (width 0.25) (layer "F.Cu") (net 1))
 (segment (start 179.955 88.265) (end 185.065 88.265) (width 0.25) (layer "F.Cu") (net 1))
 (segment (start 185.1 88.3) (end 189.2 88.3) (width 0.25) (layer "F.Cu") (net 1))
 (segment (start 193.75 86.5) (end 191.95 88.3) (width 0.25) (layer "F.Cu") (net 1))
 (segment (start 196.05 86.5) (end 193.75 86.5) (width 0.25) (layer "F.Cu") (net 1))
 (segment (start 191.95 88.3) (end 189.2 88.3) (width 0.25) (layer "F.Cu") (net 1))
 (segment (start 185.1 86.7) (end 189.2 86.7) (width 0.25) (layer "F.Cu") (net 2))
 (segment (start 185.1 86.7) (end 185.1 84.325) (width 0.25) (layer "F.Cu") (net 2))
 (segment (start 185.1 84.325) (end 184.975 84.2) (width 0.25) (layer "F.Cu") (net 2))
 (segment (start 180.93 86.7) (end 185.1 86.7) (width 0.25) (layer "F.Cu") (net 2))
 (segment (start 179.955 85.725) (end 180.93 86.7) (width 0.25) (layer "F.Cu") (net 2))
 (segment (start 186.775 74) (end 190.975 69.8) (width 0.25) (layer "F.Cu") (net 44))
 (segment (start 182.65 74) (end 186.775 74) (width 0.25) (layer "F.Cu") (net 44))
 (segment (start 184.975 73.2) (end 190.975 67.2) (width 0.25) (layer "F.Cu") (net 45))
 (segment (start 182.65 73.2) (end 184.975 73.2) (width 0.25) (layer "F.Cu") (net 45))
 (segment (start 196.05 84) (end 191.3 84) (width 0.25) (layer "F.Cu") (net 7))
 (segment (start 183.7 76.4) (end 182.65 76.4) (width 0.25) (layer "F.Cu") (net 7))
 (segment (start 191.3 84) (end 183.7 76.4) (width 0.25) (layer "F.Cu") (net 7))
 (segment (start 196.05 82.75) (end 191.25 82.75) (width 0.25) (layer "F.Cu") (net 6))
 (segment (start 191.25 82.75) (end 184.1 75.6) (width 0.25) (layer "F.Cu") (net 6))
 (segment (start 184.1 75.6) (end 182.65 75.6) (width 0.25) (layer "F.Cu") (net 6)))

